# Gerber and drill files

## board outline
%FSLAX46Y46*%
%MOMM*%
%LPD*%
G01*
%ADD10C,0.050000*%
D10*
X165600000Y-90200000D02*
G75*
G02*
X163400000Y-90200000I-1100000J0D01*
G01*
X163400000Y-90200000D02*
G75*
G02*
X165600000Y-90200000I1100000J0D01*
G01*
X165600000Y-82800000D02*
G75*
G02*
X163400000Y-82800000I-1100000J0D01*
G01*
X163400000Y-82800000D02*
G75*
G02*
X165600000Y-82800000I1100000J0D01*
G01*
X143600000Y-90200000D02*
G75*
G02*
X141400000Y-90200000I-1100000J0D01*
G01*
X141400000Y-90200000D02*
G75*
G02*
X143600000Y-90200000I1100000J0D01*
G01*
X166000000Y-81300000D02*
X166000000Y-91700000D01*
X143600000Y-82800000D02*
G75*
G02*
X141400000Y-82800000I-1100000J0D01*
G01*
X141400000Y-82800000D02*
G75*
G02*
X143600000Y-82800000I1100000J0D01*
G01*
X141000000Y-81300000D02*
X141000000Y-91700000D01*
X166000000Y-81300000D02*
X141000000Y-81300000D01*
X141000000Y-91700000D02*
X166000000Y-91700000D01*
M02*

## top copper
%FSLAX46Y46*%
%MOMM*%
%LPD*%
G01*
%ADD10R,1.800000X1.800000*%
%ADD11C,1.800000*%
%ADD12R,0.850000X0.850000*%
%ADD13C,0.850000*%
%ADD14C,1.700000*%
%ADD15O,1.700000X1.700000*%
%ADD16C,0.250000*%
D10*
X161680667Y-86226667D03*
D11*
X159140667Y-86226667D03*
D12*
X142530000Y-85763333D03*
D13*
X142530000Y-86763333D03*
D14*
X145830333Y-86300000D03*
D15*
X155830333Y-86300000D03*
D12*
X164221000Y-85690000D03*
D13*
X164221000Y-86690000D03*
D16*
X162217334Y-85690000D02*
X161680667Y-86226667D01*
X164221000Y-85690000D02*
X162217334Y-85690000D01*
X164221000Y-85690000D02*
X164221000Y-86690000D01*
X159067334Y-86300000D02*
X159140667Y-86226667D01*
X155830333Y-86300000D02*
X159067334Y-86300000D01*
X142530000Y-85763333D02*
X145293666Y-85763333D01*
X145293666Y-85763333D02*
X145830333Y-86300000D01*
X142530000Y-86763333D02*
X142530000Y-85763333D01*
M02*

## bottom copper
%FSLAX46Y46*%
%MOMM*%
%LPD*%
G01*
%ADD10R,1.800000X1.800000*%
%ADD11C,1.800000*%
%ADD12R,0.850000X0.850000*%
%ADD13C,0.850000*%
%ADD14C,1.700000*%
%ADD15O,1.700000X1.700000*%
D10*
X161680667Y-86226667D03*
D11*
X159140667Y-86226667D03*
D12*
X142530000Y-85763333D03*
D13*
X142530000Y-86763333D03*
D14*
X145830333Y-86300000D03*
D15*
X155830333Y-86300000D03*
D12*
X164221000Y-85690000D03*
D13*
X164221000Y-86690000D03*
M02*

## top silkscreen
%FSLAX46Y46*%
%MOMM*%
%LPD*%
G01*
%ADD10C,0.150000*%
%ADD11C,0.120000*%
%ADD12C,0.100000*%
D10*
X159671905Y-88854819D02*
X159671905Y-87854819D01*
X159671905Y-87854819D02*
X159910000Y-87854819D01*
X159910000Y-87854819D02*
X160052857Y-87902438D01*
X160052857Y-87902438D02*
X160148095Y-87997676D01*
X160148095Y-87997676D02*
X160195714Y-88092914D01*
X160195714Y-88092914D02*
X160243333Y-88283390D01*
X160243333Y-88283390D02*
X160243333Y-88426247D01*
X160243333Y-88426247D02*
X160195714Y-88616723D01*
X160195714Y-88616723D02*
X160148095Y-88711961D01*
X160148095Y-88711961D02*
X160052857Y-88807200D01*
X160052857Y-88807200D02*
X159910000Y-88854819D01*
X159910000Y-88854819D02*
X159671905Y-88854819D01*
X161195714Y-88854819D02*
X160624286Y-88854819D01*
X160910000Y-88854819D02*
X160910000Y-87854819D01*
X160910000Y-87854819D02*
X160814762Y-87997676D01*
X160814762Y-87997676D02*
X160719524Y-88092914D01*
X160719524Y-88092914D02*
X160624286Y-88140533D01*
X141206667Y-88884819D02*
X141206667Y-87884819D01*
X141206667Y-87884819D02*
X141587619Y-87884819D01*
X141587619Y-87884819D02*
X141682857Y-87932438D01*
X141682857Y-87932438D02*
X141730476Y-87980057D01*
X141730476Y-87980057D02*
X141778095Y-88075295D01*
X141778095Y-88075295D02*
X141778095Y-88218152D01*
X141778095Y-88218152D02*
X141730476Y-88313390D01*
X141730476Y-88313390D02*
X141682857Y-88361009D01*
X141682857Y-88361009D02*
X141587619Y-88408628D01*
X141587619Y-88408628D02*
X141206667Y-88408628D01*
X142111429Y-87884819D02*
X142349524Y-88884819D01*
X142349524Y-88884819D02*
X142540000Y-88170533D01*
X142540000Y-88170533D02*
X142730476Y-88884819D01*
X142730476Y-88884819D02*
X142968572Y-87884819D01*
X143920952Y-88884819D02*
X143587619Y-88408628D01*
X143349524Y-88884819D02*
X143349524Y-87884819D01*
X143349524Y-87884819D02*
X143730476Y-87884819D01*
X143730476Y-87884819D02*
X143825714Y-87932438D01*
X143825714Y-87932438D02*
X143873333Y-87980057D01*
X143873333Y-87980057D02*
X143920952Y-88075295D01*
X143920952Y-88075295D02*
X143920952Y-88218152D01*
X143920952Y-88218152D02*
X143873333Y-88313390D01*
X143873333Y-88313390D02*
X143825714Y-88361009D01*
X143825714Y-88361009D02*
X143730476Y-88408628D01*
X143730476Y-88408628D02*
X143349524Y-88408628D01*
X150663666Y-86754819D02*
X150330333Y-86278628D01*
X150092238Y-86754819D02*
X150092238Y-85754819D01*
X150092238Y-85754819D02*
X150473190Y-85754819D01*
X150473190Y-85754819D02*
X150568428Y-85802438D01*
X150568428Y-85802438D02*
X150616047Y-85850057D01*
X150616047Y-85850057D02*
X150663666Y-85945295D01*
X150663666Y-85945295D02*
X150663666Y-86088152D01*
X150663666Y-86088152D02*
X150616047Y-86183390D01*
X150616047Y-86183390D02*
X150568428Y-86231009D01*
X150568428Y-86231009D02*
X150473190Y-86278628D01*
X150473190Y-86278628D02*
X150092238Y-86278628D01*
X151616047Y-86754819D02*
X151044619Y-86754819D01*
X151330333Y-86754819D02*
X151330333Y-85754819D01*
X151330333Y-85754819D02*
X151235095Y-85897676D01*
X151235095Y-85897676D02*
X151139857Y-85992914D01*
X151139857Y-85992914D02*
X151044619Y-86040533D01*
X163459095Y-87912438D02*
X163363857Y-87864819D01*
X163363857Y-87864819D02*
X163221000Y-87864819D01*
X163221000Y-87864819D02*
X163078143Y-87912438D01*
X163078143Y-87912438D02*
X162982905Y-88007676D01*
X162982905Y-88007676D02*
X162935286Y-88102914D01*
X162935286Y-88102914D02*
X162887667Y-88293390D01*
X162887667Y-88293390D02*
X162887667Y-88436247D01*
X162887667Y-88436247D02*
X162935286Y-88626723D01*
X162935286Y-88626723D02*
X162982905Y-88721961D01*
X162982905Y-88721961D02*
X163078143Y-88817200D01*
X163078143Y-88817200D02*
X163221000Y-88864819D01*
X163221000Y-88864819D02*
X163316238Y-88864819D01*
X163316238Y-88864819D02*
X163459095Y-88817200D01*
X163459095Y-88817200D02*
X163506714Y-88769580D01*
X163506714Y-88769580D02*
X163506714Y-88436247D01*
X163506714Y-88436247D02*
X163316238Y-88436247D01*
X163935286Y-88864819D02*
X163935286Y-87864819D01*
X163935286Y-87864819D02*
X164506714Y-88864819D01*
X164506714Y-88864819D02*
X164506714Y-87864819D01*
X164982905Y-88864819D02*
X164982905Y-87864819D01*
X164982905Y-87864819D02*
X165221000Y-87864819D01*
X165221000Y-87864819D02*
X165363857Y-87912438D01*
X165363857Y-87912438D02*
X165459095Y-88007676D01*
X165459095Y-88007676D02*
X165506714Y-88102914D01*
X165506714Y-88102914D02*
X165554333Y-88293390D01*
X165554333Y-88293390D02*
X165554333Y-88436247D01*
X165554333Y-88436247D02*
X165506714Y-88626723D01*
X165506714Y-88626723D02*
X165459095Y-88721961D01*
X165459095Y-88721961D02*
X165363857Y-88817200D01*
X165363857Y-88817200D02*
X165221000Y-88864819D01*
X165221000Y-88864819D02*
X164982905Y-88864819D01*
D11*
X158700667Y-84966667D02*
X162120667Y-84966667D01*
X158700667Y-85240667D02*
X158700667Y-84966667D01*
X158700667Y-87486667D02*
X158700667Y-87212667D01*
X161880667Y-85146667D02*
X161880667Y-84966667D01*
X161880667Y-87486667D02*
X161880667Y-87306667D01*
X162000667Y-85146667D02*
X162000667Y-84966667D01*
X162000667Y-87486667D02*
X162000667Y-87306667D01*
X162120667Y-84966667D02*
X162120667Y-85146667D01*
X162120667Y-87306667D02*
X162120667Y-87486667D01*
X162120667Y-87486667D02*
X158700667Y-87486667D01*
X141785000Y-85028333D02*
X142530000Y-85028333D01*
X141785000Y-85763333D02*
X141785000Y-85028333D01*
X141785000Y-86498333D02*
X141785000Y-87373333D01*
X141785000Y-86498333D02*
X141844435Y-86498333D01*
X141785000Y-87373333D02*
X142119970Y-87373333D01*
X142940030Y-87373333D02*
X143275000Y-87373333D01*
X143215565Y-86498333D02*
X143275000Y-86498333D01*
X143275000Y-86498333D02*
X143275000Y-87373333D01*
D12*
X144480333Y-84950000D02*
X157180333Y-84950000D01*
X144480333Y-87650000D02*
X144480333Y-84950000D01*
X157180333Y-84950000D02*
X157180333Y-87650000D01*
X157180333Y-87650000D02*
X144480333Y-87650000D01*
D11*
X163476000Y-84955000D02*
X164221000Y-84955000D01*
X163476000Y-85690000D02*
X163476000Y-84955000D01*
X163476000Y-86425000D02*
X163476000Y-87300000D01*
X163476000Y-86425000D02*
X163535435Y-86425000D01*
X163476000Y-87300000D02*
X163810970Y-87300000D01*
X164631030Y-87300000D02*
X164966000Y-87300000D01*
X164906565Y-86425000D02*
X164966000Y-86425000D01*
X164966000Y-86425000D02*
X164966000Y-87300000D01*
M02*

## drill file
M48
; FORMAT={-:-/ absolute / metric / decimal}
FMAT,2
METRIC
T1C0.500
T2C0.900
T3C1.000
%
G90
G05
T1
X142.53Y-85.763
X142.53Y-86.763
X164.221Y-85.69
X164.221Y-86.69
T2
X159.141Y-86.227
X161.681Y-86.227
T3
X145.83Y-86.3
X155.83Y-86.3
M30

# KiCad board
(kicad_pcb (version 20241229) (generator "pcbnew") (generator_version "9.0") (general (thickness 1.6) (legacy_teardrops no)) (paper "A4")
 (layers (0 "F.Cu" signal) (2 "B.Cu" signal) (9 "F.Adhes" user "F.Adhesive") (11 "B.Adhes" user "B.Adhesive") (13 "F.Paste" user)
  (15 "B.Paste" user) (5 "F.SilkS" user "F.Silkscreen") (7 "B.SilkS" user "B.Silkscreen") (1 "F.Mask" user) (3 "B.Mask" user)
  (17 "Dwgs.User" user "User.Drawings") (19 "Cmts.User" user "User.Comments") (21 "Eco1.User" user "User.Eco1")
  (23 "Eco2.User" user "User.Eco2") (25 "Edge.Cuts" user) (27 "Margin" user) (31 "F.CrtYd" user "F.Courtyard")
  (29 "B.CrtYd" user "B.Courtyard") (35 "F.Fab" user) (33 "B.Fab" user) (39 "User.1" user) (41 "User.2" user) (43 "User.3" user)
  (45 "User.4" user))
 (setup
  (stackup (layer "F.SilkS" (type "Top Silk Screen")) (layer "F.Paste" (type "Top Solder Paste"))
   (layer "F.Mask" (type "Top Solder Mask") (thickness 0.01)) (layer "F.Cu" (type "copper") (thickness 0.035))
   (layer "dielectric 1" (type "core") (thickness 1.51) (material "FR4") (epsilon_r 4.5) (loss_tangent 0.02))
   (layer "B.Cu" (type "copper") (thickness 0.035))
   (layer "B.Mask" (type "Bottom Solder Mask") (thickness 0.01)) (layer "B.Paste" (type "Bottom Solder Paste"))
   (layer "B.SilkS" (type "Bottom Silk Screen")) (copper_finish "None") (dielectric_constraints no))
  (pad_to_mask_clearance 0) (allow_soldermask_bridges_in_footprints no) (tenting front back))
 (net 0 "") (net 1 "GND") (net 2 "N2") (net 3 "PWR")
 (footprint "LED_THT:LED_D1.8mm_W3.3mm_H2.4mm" (layer "F.Cu") (at 161.680667 86.226667 180)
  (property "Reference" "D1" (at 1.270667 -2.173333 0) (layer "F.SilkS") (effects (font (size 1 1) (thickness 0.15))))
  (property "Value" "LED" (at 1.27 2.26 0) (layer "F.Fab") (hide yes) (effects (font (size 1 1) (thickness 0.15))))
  (fp_line (start 2.98 1.26) (end -0.44 1.26) (stroke (width 0.12) (type solid)) (layer "F.SilkS"))
  (fp_line (start 2.98 0.986) (end 2.98 1.26) (stroke (width 0.12) (type solid)) (layer "F.SilkS"))
  (fp_line (start 2.98 -1.26) (end 2.98 -0.986) (stroke (width 0.12) (type solid)) (layer "F.SilkS"))
  (fp_line (start -0.2 1.08) (end -0.2 1.26) (stroke (width 0.12) (type solid)) (layer "F.SilkS"))
  (fp_line (start -0.2 -1.26) (end -0.2 -1.08) (stroke (width 0.12) (type solid)) (layer "F.SilkS"))
  (fp_line (start -0.32 1.08) (end -0.32 1.26) (stroke (width 0.12) (type solid)) (layer "F.SilkS"))
  (fp_line (start -0.32 -1.26) (end -0.32 -1.08) (stroke (width 0.12) (type solid)) (layer "F.SilkS"))
  (fp_line (start -0.44 1.26) (end -0.44 1.08) (stroke (width 0.12) (type solid)) (layer "F.SilkS"))
  (fp_line (start -0.44 -1.08) (end -0.44 -1.26) (stroke (width 0.12) (type solid)) (layer "F.SilkS"))
  (fp_line (start -0.44 -1.26) (end 2.98 -1.26) (stroke (width 0.12) (type solid)) (layer "F.SilkS"))
  (pad "1" thru_hole rect (at 0 0 180) (size 1.8 1.8) (drill 0.9) (layers "*.Cu" "*.Mask") (remove_unused_layers no) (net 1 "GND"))
  (pad "2" thru_hole circle (at 2.54 0 180) (size 1.8 1.8) (drill 0.9) (layers "*.Cu" "*.Mask") (remove_unused_layers no) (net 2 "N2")))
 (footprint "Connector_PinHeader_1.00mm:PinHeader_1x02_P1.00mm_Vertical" (layer "F.Cu") (at 142.53 85.763333)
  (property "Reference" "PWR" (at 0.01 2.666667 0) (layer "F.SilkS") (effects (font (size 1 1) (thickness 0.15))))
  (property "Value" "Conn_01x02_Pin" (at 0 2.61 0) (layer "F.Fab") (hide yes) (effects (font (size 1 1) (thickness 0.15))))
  (fp_line (start -0.745 -0.735) (end 0 -0.735) (stroke (width 0.12) (type solid)) (layer "F.SilkS"))
  (fp_line (start -0.745 0) (end -0.745 -0.735) (stroke (width 0.12) (type solid)) (layer "F.SilkS"))
  (fp_line (start -0.745 0.735) (end -0.745 1.61) (stroke (width 0.12) (type solid)) (layer "F.SilkS"))
  (fp_line (start -0.745 0.735) (end -0.685565 0.735) (stroke (width 0.12) (type solid)) (layer "F.SilkS"))
  (fp_line (start -0.745 1.61) (end -0.41003 1.61) (stroke (width 0.12) (type solid)) (layer "F.SilkS"))
  (fp_line (start 0.41003 1.61) (end 0.745 1.61) (stroke (width 0.12) (type solid)) (layer "F.SilkS"))
  (fp_line (start 0.685565 0.735) (end 0.745 0.735) (stroke (width 0.12) (type solid)) (layer "F.SilkS"))
  (fp_line (start 0.745 0.735) (end 0.745 1.61) (stroke (width 0.12) (type solid)) (layer "F.SilkS"))
  (pad "1" thru_hole rect (at 0 0) (size 0.85 0.85) (drill 0.5) (layers "*.Cu" "*.Mask") (remove_unused_layers no) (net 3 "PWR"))
  (pad "2" thru_hole circle (at 0 1) (size 0.85 0.85) (drill 0.5) (layers "*.Cu" "*.Mask") (remove_unused_layers no) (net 3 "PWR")))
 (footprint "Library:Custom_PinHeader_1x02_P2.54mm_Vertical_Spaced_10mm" (layer "F.Cu") (at 150.830333 86.3 90)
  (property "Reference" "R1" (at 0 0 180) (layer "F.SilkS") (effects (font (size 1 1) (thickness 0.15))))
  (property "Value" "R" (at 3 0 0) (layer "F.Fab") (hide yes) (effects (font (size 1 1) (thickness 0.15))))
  (fp_line (start 1.35 -6.35) (end 1.35 6.35) (stroke (width 0.1) (type default)) (layer "F.SilkS"))
  (fp_line (start -1.35 -6.35) (end 1.35 -6.35) (stroke (width 0.1) (type default)) (layer "F.SilkS"))
  (fp_line (start 1.35 6.35) (end -1.35 6.35) (stroke (width 0.1) (type default)) (layer "F.SilkS"))
  (fp_line (start -1.35 6.35) (end -1.35 -6.35) (stroke (width 0.1) (type default)) (layer "F.SilkS"))
  (pad "1" thru_hole circle (at 0 -5 90) (size 1.7 1.7) (drill 1) (layers "*.Cu" "*.Mask") (remove_unused_layers no) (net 3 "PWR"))
  (pad "2" thru_hole oval (at 0 5 90) (size 1.7 1.7) (drill 1) (layers "*.Cu" "*.Mask") (remove_unused_layers no) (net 2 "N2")))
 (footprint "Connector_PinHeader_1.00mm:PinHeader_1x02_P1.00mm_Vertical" (layer "F.Cu") (at 164.221 85.69)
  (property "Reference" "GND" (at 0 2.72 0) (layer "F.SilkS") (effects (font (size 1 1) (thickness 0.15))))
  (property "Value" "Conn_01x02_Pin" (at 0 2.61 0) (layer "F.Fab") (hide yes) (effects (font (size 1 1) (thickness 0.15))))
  (fp_line (start -0.745 -0.735) (end 0 -0.735) (stroke (width 0.12) (type solid)) (layer "F.SilkS"))
  (fp_line (start -0.745 0) (end -0.745 -0.735) (stroke (width 0.12) (type solid)) (layer "F.SilkS"))
  (fp_line (start -0.745 0.735) (end -0.745 1.61) (stroke (width 0.12) (type solid)) (layer "F.SilkS"))
  (fp_line (start -0.745 0.735) (end -0.685565 0.735) (stroke (width 0.12) (type solid)) (layer "F.SilkS"))
  (fp_line (start -0.745 1.61) (end -0.41003 1.61) (stroke (width 0.12) (type solid)) (layer "F.SilkS"))
  (fp_line (start 0.41003 1.61) (end 0.745 1.61) (stroke (width 0.12) (type solid)) (layer "F.SilkS"))
  (fp_line (start 0.685565 0.735) (end 0.745 0.735) (stroke (width 0.12) (type solid)) (layer "F.SilkS"))
  (fp_line (start 0.745 0.735) (end 0.745 1.61) (stroke (width 0.12) (type solid)) (layer "F.SilkS"))
  (pad "1" thru_hole rect (at 0 0) (size 0.85 0.85) (drill 0.5) (layers "*.Cu" "*.Mask") (remove_unused_layers no) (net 1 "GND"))
  (pad "2" thru_hole circle (at 0 1) (size 0.85 0.85) (drill 0.5) (layers "*.Cu" "*.Mask") (remove_unused_layers no) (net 1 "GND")))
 (gr_circle (center 164.5 90.2) (end 165.6 90.2) (stroke (width 0.05) (type solid)) (fill no) (layer "Edge.Cuts"))
 (gr_circle (center 164.5 82.8) (end 165.6 82.8) (stroke (width 0.05) (type solid)) (fill no) (layer "Edge.Cuts"))
 (gr_circle (center 142.5 90.2) (end 143.6 90.2) (stroke (width 0.05) (type solid)) (fill no) (layer "Edge.Cuts"))
 (gr_line (start 166 81.3) (end 166 91.7) (stroke (width 0.05) (type default)) (layer "Edge.Cuts"))
 (gr_circle (center 142.5 82.8) (end 143.6 82.8) (stroke (width 0.05) (type solid)) (fill no) (layer "Edge.Cuts"))
 (gr_line (start 141 81.3) (end 141 91.7) (stroke (width 0.05) (type default)) (layer "Edge.Cuts"))
 (gr_line (start 166 81.3) (end 141 81.3) (stroke (width 0.05) (type default)) (layer "Edge.Cuts"))
 (gr_line (start 141 91.7) (end 166 91.7) (stroke (width 0.05) (type default)) (layer "Edge.Cuts"))
 (segment (start 162.217334 85.69) (end 161.680667 86.226667) (width 0.25) (layer "F.Cu") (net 1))
 (segment (start 164.221 85.69) (end 162.217334 85.69) (width 0.25) (layer "F.Cu") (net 1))
 (segment (start 164.221 85.69) (end 164.221 86.69) (width 0.25) (layer "F.Cu") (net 1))
 (segment (start 159.067334 86.3) (end 159.140667 86.226667) (width 0.25) (layer "F.Cu") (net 2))
 (segment (start 155.830333 86.3) (end 159.067334 86.3) (width 0.25) (layer "F.Cu") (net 2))
 (segment (start 142.53 85.763333) (end 145.293666 85.763333) (width 0.25) (layer "F.Cu") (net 3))
 (segment (start 145.293666 85.763333) (end 145.830333 86.3) (width 0.25) (layer "F.Cu") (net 3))
 (segment (start 142.53 86.763333) (end 142.53 85.763333) (width 0.25) (layer "F.Cu") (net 3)))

